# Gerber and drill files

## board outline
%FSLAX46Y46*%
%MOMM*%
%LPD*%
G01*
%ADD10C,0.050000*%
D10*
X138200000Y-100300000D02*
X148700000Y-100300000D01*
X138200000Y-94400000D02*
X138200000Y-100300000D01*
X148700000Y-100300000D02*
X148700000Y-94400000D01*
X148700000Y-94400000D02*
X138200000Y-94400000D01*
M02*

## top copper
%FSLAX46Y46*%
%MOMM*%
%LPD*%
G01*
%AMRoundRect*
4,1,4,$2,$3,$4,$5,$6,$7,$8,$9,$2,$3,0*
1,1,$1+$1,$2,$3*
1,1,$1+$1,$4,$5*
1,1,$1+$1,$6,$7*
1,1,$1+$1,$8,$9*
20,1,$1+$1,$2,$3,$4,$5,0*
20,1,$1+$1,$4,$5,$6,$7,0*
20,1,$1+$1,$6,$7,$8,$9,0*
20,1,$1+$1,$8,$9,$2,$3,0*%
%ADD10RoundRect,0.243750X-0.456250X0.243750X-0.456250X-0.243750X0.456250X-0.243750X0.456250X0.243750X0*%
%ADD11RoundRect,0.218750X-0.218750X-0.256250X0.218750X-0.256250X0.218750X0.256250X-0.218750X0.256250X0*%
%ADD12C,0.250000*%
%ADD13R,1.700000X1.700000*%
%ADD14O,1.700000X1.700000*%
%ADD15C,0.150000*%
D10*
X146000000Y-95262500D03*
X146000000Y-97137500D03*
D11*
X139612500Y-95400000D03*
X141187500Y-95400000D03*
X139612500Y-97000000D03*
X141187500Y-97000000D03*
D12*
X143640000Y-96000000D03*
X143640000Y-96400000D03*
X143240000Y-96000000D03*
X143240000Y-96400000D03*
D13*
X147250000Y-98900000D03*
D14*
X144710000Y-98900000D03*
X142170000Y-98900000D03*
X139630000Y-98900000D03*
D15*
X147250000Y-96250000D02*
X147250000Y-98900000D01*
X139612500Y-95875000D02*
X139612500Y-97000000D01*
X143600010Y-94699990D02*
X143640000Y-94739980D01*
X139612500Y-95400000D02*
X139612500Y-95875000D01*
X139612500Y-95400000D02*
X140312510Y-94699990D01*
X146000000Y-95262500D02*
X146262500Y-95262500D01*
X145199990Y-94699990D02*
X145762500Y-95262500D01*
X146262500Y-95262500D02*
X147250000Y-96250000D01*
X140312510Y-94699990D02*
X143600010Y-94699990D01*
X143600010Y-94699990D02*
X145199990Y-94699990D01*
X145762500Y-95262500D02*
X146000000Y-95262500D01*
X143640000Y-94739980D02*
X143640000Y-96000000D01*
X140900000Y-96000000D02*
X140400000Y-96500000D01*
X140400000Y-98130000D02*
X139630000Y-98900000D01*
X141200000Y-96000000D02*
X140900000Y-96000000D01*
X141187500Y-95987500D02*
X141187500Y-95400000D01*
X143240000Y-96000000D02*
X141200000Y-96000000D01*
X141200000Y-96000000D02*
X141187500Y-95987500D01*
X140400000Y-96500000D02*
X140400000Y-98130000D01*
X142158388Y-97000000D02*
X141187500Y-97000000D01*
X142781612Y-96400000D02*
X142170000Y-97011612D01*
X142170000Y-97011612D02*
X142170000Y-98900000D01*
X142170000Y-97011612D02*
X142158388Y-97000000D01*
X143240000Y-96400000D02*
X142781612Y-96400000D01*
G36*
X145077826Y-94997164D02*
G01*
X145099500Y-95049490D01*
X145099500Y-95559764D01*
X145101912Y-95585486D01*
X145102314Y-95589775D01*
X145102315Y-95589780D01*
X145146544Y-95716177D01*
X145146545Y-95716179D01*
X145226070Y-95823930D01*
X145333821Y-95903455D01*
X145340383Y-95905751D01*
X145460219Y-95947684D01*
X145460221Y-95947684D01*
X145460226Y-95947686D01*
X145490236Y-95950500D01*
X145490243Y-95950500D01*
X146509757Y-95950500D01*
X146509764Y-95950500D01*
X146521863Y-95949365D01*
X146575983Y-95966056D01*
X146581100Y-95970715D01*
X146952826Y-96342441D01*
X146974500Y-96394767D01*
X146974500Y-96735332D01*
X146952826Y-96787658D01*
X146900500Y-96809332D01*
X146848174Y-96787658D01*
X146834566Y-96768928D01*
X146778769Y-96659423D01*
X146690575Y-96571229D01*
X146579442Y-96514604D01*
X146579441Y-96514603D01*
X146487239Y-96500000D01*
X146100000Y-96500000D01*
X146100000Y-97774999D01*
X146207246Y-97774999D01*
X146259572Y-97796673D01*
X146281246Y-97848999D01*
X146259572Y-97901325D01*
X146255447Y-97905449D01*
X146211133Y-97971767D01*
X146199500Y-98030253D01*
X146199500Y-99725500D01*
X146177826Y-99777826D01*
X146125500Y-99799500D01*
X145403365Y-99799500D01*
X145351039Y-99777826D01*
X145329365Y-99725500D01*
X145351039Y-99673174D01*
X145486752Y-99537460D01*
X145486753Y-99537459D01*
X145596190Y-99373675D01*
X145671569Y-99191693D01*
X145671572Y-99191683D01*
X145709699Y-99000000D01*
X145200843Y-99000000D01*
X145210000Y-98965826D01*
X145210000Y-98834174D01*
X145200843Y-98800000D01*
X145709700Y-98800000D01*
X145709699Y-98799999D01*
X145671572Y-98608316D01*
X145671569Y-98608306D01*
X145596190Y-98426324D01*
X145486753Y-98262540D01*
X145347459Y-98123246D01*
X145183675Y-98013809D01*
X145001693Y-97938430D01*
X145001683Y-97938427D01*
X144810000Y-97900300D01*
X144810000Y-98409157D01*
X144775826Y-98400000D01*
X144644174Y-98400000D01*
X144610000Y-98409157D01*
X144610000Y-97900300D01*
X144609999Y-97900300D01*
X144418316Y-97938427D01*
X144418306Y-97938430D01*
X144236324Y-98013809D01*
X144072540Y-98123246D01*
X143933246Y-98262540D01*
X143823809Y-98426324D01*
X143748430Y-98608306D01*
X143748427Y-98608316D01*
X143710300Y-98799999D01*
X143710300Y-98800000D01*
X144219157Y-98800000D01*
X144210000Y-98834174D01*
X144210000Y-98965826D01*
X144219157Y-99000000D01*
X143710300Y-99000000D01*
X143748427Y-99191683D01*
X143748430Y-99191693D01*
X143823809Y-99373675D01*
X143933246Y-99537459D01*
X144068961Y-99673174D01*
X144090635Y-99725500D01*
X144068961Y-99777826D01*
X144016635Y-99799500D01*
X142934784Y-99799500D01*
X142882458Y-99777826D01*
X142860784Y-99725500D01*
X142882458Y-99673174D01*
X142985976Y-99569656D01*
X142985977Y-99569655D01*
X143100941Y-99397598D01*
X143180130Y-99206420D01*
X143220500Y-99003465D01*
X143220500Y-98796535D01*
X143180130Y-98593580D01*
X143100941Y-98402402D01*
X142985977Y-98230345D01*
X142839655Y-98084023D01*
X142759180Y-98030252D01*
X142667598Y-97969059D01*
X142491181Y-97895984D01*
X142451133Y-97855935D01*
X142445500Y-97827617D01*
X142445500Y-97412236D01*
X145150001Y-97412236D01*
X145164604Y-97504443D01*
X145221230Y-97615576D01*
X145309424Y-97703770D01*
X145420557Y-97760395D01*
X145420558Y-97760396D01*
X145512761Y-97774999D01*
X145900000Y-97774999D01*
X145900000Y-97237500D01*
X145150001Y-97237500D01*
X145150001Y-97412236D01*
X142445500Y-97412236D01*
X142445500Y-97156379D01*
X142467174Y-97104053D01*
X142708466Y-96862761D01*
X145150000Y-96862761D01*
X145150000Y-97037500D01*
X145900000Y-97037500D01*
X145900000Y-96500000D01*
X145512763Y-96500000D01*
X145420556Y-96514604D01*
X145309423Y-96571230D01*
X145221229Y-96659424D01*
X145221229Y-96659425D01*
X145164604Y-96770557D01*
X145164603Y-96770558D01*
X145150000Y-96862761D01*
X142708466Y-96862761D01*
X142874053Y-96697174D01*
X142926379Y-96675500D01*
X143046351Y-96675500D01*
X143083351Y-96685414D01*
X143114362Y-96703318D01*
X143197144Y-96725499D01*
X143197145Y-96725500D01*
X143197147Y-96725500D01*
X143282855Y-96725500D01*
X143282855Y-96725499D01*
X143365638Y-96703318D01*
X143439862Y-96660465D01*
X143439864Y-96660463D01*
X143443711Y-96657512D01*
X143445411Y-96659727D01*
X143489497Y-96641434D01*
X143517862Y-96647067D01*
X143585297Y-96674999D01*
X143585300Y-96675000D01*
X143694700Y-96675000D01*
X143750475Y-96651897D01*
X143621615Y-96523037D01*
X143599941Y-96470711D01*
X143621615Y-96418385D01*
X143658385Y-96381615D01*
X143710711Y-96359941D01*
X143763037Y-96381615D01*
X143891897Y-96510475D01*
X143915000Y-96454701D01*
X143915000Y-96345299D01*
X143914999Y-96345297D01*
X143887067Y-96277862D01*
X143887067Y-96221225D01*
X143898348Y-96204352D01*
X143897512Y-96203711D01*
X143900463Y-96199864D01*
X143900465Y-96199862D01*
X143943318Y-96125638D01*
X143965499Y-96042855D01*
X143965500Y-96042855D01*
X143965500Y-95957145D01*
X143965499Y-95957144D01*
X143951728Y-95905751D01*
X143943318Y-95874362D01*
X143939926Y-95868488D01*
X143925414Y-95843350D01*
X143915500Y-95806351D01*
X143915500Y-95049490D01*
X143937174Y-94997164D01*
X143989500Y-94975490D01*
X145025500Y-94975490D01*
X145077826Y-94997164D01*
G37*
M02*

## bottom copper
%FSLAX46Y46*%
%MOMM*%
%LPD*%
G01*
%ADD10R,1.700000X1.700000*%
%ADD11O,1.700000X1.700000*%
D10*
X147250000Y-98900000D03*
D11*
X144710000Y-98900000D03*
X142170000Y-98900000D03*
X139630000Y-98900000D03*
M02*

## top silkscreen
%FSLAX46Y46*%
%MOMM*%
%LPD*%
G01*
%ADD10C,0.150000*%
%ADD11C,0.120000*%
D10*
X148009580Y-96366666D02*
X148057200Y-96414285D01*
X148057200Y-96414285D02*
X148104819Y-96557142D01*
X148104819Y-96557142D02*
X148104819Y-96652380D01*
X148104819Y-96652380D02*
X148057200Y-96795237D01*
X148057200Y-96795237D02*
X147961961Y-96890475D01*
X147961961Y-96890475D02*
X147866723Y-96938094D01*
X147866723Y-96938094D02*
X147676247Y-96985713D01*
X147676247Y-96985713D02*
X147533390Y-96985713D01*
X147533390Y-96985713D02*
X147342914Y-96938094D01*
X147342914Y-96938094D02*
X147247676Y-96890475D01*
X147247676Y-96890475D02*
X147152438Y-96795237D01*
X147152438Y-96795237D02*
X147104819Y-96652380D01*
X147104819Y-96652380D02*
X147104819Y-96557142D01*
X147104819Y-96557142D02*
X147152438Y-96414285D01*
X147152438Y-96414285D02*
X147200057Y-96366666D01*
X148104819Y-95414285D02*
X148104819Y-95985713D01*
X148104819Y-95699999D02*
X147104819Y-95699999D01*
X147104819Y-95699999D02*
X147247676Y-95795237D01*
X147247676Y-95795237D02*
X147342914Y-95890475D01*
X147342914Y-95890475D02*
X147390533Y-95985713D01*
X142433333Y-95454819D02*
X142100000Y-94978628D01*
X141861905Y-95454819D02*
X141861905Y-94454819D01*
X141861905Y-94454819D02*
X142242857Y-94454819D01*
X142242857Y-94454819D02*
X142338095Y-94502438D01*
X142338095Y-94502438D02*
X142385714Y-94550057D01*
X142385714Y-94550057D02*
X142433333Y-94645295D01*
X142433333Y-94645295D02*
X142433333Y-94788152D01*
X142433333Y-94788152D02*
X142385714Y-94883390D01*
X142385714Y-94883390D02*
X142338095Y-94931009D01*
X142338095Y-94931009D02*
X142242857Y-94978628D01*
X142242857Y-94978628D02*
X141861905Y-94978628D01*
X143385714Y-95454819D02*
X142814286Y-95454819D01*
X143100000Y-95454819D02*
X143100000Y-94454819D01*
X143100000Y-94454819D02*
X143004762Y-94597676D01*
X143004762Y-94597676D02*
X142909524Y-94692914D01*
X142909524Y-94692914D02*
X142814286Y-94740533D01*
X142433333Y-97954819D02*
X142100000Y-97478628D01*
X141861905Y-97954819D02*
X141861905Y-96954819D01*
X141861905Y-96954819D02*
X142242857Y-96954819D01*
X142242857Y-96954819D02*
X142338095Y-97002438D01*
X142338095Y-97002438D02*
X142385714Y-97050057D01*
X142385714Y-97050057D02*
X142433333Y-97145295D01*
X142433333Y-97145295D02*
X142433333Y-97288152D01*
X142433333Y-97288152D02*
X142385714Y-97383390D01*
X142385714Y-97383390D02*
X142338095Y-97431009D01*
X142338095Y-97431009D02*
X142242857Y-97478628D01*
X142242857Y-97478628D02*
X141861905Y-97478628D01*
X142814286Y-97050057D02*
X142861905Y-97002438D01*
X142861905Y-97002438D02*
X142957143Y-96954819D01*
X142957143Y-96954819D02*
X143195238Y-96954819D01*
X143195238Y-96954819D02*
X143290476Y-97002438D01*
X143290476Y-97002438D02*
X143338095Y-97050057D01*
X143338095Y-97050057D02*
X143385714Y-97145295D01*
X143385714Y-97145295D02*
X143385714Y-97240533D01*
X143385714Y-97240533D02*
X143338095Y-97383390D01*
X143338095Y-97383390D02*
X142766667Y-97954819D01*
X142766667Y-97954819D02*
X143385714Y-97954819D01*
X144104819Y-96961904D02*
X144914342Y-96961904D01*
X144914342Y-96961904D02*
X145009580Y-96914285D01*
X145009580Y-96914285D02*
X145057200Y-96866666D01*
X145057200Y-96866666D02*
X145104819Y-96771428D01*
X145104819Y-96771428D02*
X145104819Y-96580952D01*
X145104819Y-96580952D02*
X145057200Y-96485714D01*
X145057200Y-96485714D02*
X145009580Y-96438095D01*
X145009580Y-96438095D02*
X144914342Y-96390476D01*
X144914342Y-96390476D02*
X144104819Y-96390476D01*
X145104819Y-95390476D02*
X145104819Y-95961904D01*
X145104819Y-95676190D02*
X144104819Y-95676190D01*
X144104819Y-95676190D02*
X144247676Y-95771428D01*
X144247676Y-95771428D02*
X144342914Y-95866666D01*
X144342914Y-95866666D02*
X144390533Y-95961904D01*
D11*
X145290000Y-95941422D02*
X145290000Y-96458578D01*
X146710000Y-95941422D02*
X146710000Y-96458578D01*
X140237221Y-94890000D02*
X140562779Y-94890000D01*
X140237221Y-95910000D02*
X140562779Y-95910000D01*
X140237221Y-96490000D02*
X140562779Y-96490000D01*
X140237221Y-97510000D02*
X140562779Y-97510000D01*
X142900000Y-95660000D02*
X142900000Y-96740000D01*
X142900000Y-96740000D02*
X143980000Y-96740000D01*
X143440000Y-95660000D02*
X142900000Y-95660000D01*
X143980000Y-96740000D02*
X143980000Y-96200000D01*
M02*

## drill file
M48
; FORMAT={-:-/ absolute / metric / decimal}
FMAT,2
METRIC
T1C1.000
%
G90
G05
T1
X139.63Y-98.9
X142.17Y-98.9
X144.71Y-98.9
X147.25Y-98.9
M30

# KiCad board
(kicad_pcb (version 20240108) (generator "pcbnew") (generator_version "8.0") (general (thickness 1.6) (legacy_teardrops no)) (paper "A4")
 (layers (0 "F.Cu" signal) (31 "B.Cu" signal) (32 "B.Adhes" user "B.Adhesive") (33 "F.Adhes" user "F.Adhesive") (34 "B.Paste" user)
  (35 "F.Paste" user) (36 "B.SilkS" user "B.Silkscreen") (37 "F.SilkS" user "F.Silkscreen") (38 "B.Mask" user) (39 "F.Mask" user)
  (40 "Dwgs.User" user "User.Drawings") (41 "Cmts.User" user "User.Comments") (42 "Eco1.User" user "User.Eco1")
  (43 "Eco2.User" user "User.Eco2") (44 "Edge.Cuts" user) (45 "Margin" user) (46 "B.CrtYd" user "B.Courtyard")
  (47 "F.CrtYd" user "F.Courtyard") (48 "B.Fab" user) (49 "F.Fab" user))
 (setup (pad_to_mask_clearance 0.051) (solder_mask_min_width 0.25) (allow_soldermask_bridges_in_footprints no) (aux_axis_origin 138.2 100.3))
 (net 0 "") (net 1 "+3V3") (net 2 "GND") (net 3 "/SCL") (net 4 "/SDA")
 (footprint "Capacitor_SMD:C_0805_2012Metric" (layer "F.Cu") (at 146 96.2 -90)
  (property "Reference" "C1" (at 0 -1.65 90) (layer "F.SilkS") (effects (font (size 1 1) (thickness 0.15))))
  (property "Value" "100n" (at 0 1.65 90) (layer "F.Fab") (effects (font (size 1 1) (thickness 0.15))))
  (fp_line (start -0.258578 0.71) (end 0.258578 0.71) (stroke (width 0.12) (type solid)) (layer "F.SilkS"))
  (fp_line (start -0.258578 -0.71) (end 0.258578 -0.71) (stroke (width 0.12) (type solid)) (layer "F.SilkS"))
  (pad "1" smd roundrect (at -0.9375 0 270) (size 0.975 1.4) (layers "F.Cu" "F.Paste" "F.Mask") (roundrect_rratio 0.25) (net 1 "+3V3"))
  (pad "2" smd roundrect (at 0.9375 0 270) (size 0.975 1.4) (layers "F.Cu" "F.Paste" "F.Mask") (roundrect_rratio 0.25) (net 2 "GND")))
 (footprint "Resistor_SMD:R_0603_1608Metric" (layer "F.Cu") (at 140.4 95.4)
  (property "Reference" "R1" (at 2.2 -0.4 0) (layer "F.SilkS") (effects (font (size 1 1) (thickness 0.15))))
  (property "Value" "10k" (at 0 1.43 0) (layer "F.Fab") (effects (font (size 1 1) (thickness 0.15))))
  (fp_line (start -0.162779 -0.51) (end 0.162779 -0.51) (stroke (width 0.12) (type solid)) (layer "F.SilkS"))
  (fp_line (start -0.162779 0.51) (end 0.162779 0.51) (stroke (width 0.12) (type solid)) (layer "F.SilkS"))
  (pad "1" smd roundrect (at -0.7875 0) (size 0.875 0.95) (layers "F.Cu" "F.Paste" "F.Mask") (roundrect_rratio 0.25) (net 1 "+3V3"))
  (pad "2" smd roundrect (at 0.7875 0) (size 0.875 0.95) (layers "F.Cu" "F.Paste" "F.Mask") (roundrect_rratio 0.25) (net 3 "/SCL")))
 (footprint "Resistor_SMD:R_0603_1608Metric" (layer "F.Cu") (at 140.4 97)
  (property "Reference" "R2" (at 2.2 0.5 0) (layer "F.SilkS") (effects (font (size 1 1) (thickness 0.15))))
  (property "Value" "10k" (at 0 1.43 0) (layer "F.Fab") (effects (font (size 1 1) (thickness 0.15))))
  (fp_line (start -0.162779 -0.51) (end 0.162779 -0.51) (stroke (width 0.12) (type solid)) (layer "F.SilkS"))
  (fp_line (start -0.162779 0.51) (end 0.162779 0.51) (stroke (width 0.12) (type solid)) (layer "F.SilkS"))
  (pad "1" smd roundrect (at -0.7875 0) (size 0.875 0.95) (layers "F.Cu" "F.Paste" "F.Mask") (roundrect_rratio 0.25) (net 1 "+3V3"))
  (pad "2" smd roundrect (at 0.7875 0) (size 0.875 0.95) (layers "F.Cu" "F.Paste" "F.Mask") (roundrect_rratio 0.25) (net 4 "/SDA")))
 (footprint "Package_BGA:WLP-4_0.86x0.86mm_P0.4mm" (layer "F.Cu") (at 143.44 96.2 -90)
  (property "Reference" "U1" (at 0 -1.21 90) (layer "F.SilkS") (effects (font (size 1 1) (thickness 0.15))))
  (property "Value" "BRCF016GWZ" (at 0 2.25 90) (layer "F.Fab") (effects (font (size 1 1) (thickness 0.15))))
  (fp_line (start -0.54 0.54) (end 0.54 0.54) (stroke (width 0.12) (type solid)) (layer "F.SilkS"))
  (fp_line (start 0.54 0.54) (end 0.54 -0.54) (stroke (width 0.12) (type solid)) (layer "F.SilkS"))
  (fp_line (start -0.54 0) (end -0.54 0.54) (stroke (width 0.12) (type solid)) (layer "F.SilkS"))
  (fp_line (start 0.54 -0.54) (end 0 -0.54) (stroke (width 0.12) (type solid)) (layer "F.SilkS"))
  (pad "A1" smd circle (at -0.2 -0.2 270) (size 0.25 0.25) (layers "F.Cu" "F.Paste" "F.Mask") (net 1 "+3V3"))
  (pad "A2" smd circle (at 0.2 -0.2 270) (size 0.25 0.25) (layers "F.Cu" "F.Paste" "F.Mask") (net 2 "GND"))
  (pad "B1" smd circle (at -0.2 0.2 270) (size 0.25 0.25) (layers "F.Cu" "F.Paste" "F.Mask") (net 3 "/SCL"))
  (pad "B2" smd circle (at 0.2 0.2 270) (size 0.25 0.25) (layers "F.Cu" "F.Paste" "F.Mask") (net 4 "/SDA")))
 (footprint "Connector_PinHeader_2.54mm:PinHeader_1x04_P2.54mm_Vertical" (layer "B.Cu") (at 147.25 98.9 90)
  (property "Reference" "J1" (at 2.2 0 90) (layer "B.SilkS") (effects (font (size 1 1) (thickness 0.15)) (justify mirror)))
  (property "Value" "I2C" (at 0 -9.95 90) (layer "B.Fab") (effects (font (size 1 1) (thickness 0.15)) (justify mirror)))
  (pad "1" thru_hole rect (at 0 0 90) (size 1.7 1.7) (drill 1) (layers "*.Cu" "*.Mask") (remove_unused_layers no) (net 1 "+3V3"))
  (pad "2" thru_hole oval (at 0 -2.54 90) (size 1.7 1.7) (drill 1) (layers "*.Cu" "*.Mask") (remove_unused_layers no) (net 2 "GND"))
  (pad "3" thru_hole oval (at 0 -5.08 90) (size 1.7 1.7) (drill 1) (layers "*.Cu" "*.Mask") (remove_unused_layers no) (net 4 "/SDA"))
  (pad "4" thru_hole oval (at 0 -7.62 90) (size 1.7 1.7) (drill 1) (layers "*.Cu" "*.Mask") (remove_unused_layers no) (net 3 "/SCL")))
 (gr_line (start 138.2 100.3) (end 148.7 100.3) (stroke (width 0.05) (type solid)) (layer "Edge.Cuts"))
 (gr_line (start 138.2 94.4) (end 138.2 100.3) (stroke (width 0.05) (type solid)) (layer "Edge.Cuts"))
 (gr_line (start 148.7 100.3) (end 148.7 94.4) (stroke (width 0.05) (type solid)) (layer "Edge.Cuts"))
 (gr_line (start 148.7 94.4) (end 138.2 94.4) (stroke (width 0.05) (type solid)) (layer "Edge.Cuts"))
 (segment (start 147.25 96.25) (end 147.25 98.9) (width 0.15) (layer "F.Cu") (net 1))
 (segment (start 139.6125 95.875) (end 139.6125 97) (width 0.15) (layer "F.Cu") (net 1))
 (segment (start 143.60001 94.69999) (end 143.64 94.73998) (width 0.15) (layer "F.Cu") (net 1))
 (segment (start 139.6125 95.4) (end 139.6125 95.875) (width 0.15) (layer "F.Cu") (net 1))
 (segment (start 139.6125 95.4) (end 140.31251 94.69999) (width 0.15) (layer "F.Cu") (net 1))
 (segment (start 146 95.2625) (end 146.2625 95.2625) (width 0.15) (layer "F.Cu") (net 1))
 (segment (start 145.19999 94.69999) (end 145.7625 95.2625) (width 0.15) (layer "F.Cu") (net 1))
 (segment (start 146.2625 95.2625) (end 147.25 96.25) (width 0.15) (layer "F.Cu") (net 1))
 (segment (start 140.31251 94.69999) (end 143.60001 94.69999) (width 0.15) (layer "F.Cu") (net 1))
 (segment (start 143.60001 94.69999) (end 145.19999 94.69999) (width 0.15) (layer "F.Cu") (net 1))
 (segment (start 145.7625 95.2625) (end 146 95.2625) (width 0.15) (layer "F.Cu") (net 1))
 (segment (start 143.64 94.73998) (end 143.64 96) (width 0.15) (layer "F.Cu") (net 1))
 (segment (start 140.9 96) (end 140.4 96.5) (width 0.15) (layer "F.Cu") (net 3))
 (segment (start 140.4 98.13) (end 139.63 98.9) (width 0.15) (layer "F.Cu") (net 3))
 (segment (start 141.2 96) (end 140.9 96) (width 0.15) (layer "F.Cu") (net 3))
 (segment (start 141.1875 95.9875) (end 141.1875 95.4) (width 0.15) (layer "F.Cu") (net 3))
 (segment (start 143.24 96) (end 141.2 96) (width 0.15) (layer "F.Cu") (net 3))
 (segment (start 141.2 96) (end 141.1875 95.9875) (width 0.15) (layer "F.Cu") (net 3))
 (segment (start 140.4 96.5) (end 140.4 98.13) (width 0.15) (layer "F.Cu") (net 3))
 (segment (start 142.158388 97) (end 141.1875 97) (width 0.15) (layer "F.Cu") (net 4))
 (segment (start 142.781612 96.4) (end 142.17 97.011612) (width 0.15) (layer "F.Cu") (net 4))
 (segment (start 142.17 97.011612) (end 142.17 98.9) (width 0.15) (layer "F.Cu") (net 4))
 (segment (start 142.17 97.011612) (end 142.158388 97) (width 0.15) (layer "F.Cu") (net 4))
 (segment (start 143.24 96.4) (end 142.781612 96.4) (width 0.15) (layer "F.Cu") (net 4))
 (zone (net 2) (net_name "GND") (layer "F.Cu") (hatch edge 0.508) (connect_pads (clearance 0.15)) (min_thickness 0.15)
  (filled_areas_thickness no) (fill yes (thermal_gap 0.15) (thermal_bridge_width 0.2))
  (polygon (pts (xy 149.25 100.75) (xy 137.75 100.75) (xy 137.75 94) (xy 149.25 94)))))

